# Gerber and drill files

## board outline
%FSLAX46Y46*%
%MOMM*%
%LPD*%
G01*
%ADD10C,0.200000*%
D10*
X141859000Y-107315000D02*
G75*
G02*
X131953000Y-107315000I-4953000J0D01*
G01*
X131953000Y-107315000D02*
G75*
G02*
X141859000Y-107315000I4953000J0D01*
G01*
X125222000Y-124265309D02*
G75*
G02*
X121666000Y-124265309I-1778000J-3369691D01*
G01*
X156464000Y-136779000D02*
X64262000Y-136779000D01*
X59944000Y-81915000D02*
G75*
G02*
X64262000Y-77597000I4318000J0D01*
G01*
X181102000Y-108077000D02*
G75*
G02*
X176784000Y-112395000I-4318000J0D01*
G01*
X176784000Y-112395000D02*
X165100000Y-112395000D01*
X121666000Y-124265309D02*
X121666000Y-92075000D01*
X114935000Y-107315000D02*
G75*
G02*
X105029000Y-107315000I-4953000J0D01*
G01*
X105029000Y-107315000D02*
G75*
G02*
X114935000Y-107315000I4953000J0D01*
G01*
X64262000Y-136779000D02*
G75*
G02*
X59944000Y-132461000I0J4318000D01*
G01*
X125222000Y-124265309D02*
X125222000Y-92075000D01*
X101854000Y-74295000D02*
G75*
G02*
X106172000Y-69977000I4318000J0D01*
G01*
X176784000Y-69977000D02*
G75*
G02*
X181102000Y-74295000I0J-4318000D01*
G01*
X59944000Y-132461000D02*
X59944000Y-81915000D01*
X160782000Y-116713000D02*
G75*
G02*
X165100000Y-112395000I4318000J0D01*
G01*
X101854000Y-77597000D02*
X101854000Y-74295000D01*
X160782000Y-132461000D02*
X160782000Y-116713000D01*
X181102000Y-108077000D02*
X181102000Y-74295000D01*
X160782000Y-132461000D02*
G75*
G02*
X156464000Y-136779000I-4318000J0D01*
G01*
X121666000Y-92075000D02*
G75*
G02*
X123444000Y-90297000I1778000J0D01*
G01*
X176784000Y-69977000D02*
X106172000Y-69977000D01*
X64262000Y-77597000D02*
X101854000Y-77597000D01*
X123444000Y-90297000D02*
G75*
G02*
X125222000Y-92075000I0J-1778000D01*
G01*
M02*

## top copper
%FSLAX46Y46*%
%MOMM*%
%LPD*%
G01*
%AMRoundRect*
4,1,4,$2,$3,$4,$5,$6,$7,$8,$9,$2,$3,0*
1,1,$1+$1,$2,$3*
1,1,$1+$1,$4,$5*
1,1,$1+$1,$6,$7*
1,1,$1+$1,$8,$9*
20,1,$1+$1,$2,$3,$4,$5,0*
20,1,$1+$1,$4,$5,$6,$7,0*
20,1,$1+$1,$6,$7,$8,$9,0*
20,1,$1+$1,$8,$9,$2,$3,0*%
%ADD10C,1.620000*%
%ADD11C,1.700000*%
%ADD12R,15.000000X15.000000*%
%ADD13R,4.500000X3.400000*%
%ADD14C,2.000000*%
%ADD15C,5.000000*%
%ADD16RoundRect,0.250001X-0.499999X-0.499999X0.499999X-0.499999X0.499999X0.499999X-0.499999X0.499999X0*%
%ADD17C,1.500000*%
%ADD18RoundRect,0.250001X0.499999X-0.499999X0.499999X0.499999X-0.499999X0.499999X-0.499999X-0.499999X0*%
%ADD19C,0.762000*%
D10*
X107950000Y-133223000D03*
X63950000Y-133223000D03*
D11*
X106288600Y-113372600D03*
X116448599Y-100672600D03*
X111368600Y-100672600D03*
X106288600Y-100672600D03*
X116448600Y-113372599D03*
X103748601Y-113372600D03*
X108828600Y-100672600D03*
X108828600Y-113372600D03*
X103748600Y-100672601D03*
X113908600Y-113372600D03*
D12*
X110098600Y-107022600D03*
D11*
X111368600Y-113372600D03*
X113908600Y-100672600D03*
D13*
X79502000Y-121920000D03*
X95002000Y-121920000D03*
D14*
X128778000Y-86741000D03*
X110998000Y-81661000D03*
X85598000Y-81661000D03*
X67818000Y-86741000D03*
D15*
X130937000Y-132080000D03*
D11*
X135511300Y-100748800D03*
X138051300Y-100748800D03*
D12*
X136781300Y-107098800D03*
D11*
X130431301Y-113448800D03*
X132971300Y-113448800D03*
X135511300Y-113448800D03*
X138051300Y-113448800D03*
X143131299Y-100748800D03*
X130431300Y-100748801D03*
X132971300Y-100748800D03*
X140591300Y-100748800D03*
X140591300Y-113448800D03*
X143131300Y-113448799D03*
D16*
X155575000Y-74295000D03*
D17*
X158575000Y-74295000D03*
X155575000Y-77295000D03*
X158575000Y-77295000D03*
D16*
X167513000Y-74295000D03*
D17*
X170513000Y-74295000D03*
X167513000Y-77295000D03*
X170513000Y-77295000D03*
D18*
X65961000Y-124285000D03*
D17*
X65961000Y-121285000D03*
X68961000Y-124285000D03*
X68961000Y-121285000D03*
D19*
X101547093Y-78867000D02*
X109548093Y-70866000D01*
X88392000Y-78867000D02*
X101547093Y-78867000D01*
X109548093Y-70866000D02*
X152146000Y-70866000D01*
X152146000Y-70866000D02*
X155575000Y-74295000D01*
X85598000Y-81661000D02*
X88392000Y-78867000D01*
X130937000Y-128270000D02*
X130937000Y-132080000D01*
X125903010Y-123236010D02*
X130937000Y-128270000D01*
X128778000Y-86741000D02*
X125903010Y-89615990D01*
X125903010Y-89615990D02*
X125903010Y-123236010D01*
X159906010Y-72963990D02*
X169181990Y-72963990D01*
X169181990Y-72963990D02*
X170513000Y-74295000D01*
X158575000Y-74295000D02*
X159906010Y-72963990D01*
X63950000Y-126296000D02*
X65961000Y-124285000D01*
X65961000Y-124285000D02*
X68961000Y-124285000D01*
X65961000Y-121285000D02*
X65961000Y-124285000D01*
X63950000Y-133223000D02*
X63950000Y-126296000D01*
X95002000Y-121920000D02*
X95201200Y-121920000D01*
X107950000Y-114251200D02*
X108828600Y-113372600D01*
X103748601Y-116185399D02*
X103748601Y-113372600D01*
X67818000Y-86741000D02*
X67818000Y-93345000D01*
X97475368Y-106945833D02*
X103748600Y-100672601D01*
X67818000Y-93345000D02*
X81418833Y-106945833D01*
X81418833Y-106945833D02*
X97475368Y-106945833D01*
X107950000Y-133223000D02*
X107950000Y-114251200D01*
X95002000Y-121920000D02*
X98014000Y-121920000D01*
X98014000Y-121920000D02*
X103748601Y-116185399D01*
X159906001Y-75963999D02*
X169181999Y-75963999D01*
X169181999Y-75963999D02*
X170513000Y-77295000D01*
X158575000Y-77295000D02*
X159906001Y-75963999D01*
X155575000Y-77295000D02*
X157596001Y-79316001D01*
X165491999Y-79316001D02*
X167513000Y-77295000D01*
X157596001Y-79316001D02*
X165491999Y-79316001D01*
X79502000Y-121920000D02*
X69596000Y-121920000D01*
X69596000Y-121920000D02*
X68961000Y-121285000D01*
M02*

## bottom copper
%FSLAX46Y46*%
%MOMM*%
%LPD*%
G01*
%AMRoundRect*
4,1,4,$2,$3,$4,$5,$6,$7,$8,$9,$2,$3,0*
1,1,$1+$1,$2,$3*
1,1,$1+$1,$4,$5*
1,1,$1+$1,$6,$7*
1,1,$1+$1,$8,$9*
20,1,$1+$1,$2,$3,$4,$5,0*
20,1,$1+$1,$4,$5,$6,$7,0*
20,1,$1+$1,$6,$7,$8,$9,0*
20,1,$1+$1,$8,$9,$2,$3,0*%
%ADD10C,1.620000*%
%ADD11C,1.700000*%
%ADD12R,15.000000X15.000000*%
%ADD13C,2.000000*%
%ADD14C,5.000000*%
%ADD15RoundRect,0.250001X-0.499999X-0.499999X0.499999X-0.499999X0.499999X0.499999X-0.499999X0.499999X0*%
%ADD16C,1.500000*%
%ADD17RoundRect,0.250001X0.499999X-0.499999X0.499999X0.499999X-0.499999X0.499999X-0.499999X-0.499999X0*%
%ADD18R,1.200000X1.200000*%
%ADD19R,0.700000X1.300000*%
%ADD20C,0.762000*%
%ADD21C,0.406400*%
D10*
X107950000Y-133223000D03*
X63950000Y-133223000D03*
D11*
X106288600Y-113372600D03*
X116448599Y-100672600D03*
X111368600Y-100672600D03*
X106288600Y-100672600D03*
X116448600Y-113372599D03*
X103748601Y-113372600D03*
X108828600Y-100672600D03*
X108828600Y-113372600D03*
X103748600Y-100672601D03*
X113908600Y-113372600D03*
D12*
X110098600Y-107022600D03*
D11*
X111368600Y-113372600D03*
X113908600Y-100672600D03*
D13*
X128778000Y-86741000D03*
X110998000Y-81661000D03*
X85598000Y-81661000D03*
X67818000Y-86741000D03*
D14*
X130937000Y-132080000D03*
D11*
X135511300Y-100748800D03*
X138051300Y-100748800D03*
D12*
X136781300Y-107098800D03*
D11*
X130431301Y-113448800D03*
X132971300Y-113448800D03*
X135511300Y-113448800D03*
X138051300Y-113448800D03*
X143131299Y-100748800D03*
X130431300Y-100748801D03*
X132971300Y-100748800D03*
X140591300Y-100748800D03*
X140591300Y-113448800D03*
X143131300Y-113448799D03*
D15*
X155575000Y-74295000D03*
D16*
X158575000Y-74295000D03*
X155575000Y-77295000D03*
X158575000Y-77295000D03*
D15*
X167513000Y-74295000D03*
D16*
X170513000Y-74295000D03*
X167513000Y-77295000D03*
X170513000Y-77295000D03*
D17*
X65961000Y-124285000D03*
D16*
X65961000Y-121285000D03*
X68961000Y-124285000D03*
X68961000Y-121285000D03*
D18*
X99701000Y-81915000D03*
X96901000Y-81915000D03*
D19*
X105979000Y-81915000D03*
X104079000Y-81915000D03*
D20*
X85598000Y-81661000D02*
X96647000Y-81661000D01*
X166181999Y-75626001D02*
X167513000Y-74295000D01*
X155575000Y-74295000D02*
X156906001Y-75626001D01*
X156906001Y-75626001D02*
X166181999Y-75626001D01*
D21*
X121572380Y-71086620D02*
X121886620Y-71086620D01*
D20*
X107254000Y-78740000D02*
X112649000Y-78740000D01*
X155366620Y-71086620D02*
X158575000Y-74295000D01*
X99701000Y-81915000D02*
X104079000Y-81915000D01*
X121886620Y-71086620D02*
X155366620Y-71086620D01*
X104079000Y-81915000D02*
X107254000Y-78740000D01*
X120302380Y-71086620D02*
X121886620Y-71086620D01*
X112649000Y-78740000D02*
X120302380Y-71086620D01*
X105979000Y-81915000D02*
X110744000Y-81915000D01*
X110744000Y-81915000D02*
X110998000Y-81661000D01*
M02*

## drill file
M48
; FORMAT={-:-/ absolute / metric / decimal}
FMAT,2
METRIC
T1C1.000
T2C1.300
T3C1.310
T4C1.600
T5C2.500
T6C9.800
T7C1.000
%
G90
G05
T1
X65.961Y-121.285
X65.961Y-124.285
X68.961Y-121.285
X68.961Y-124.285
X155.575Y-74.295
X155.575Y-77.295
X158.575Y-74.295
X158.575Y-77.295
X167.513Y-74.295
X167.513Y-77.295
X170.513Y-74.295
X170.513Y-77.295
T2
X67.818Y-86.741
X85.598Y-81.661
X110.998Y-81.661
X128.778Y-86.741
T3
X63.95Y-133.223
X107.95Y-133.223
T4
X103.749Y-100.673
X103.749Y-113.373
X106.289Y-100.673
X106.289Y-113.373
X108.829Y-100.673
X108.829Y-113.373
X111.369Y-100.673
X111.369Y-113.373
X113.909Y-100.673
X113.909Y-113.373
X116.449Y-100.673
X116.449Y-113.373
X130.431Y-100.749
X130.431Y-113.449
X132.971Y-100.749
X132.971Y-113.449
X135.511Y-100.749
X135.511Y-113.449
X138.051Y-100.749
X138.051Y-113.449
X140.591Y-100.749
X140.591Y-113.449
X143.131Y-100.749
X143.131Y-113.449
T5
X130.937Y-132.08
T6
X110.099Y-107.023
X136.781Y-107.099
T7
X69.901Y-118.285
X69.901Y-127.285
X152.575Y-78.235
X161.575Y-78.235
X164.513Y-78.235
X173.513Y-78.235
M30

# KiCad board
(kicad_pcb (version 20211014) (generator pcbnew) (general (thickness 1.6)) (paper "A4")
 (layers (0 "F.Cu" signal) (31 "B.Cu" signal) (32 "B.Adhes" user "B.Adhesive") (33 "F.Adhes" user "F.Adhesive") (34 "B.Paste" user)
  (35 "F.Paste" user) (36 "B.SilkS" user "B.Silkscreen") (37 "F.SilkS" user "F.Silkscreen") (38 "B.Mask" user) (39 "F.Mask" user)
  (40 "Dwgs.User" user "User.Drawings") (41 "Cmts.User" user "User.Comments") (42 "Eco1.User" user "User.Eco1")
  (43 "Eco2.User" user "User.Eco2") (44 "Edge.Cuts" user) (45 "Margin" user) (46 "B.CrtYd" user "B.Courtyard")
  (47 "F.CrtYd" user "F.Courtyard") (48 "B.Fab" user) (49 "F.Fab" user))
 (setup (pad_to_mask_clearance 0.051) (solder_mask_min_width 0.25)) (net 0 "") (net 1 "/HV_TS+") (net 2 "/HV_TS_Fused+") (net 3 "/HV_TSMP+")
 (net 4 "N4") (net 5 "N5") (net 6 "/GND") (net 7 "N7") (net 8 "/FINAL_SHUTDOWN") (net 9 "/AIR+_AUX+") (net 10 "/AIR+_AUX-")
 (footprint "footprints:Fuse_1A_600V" (layer "F.Cu") (at 107.95 133.223 180)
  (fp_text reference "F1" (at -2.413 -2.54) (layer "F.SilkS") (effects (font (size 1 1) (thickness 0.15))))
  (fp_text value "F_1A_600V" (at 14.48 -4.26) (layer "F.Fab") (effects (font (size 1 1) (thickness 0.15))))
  (pad "1" thru_hole circle locked (at 0 0 180) (size 1.62 1.62) (drill 1.31) (layers *.Cu *.Mask) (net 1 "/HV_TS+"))
  (pad "2" thru_hole circle locked (at 44 0 180) (size 1.62 1.62) (drill 1.31) (layers *.Cu *.Mask) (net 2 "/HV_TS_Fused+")))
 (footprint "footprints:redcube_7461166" (layer "F.Cu") (at 110.0986 107.0226)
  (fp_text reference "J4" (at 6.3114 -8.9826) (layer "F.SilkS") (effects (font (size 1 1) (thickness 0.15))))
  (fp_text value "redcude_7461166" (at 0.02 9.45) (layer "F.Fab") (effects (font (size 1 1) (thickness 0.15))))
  (pad "1" thru_hole circle locked (at -3.81 6.35) (size 1.7 1.7) (drill 1.6) (layers *.Cu *.Mask) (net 1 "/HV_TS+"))
  (pad "1" thru_hole circle locked (at 6.349999 -6.35) (size 1.7 1.7) (drill 1.6) (layers *.Cu *.Mask) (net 1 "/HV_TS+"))
  (pad "1" thru_hole circle locked (at 1.27 -6.35) (size 1.7 1.7) (drill 1.6) (layers *.Cu *.Mask) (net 1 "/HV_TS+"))
  (pad "1" thru_hole circle locked (at -3.81 -6.35) (size 1.7 1.7) (drill 1.6) (layers *.Cu *.Mask) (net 1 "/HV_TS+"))
  (pad "1" thru_hole circle locked (at 6.35 6.349999) (size 1.7 1.7) (drill 1.6) (layers *.Cu *.Mask) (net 1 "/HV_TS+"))
  (pad "1" thru_hole circle locked (at -6.349999 6.35) (size 1.7 1.7) (drill 1.6) (layers *.Cu *.Mask) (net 1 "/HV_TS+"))
  (pad "1" thru_hole circle locked (at -1.27 -6.35) (size 1.7 1.7) (drill 1.6) (layers *.Cu *.Mask) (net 1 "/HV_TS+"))
  (pad "1" thru_hole circle locked (at -1.27 6.35) (size 1.7 1.7) (drill 1.6) (layers *.Cu *.Mask) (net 1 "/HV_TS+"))
  (pad "1" thru_hole circle locked (at -6.35 -6.349999) (size 1.7 1.7) (drill 1.6) (layers *.Cu *.Mask) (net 1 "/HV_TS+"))
  (pad "1" thru_hole circle locked (at 3.81 6.35) (size 1.7 1.7) (drill 1.6) (layers *.Cu *.Mask) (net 1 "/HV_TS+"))
  (pad "1" thru_hole rect locked (at 0 0) (size 15 15) (drill 9.8) (layers *.Cu *.Mask) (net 1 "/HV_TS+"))
  (pad "1" thru_hole circle locked (at 1.27 6.35) (size 1.7 1.7) (drill 1.6) (layers *.Cu *.Mask) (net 1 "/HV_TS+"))
  (pad "1" thru_hole circle locked (at 3.81 -6.35) (size 1.7 1.7) (drill 1.6) (layers *.Cu *.Mask) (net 1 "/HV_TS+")))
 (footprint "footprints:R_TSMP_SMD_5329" (layer "F.Cu") (at 87.122 121.92)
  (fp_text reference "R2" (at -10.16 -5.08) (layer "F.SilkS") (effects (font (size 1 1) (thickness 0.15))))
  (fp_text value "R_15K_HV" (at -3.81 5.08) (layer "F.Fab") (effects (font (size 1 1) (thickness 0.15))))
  (pad "1" smd rect locked (at -7.62 0) (size 4.5 3.4) (layers "F.Cu" "F.Paste" "F.Mask") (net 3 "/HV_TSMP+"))
  (pad "2" smd rect locked (at 7.88 0) (size 4.5 3.4) (layers "F.Cu" "F.Paste" "F.Mask") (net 1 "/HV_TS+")))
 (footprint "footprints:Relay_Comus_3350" (layer "F.Cu") (at 64.008 94.234)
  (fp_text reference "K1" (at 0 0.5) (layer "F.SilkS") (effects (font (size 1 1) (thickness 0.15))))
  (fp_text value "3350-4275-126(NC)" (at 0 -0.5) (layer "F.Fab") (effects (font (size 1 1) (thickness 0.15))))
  (pad "1" thru_hole circle locked (at 64.77 -7.493) (size 2 2) (drill 1.3) (layers *.Cu *.Mask) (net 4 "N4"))
  (pad "2" thru_hole circle locked (at 46.99 -12.573) (size 2 2) (drill 1.3) (layers *.Cu *.Mask) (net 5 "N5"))
  (pad "3" thru_hole circle locked (at 21.59 -12.573) (size 2 2) (drill 1.3) (layers *.Cu *.Mask) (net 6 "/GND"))
  (pad "4" thru_hole circle locked (at 3.81 -7.493) (size 2 2) (drill 1.3) (layers *.Cu *.Mask) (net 1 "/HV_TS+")))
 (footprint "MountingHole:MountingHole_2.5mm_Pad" (layer "F.Cu") (at 130.937 132.08 -90)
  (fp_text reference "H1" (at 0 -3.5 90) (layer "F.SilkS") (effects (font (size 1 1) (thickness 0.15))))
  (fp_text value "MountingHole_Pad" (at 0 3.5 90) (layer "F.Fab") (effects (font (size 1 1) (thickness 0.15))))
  (pad "1" thru_hole circle (at 0 0 270) (size 5 5) (drill 2.5) (layers *.Cu *.Mask) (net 4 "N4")))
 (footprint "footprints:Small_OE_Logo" (layer "F.Cu") (at 153.416 107.188)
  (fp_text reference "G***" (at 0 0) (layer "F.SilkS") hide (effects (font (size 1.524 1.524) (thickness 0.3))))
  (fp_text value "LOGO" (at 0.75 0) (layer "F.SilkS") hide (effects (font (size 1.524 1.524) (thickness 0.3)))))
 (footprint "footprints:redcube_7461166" (layer "F.Cu") (at 136.7813 107.0988)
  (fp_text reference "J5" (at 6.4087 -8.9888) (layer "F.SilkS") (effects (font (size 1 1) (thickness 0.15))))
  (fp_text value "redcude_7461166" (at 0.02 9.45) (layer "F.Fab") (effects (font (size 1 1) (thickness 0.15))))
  (pad "1" thru_hole circle locked (at -1.27 -6.35) (size 1.7 1.7) (drill 1.6) (layers *.Cu *.Mask) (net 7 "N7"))
  (pad "1" thru_hole circle locked (at 1.27 -6.35) (size 1.7 1.7) (drill 1.6) (layers *.Cu *.Mask) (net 7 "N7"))
  (pad "1" thru_hole rect locked (at 0 0) (size 15 15) (drill 9.8) (layers *.Cu *.Mask) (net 7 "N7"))
  (pad "1" thru_hole circle locked (at -6.349999 6.35) (size 1.7 1.7) (drill 1.6) (layers *.Cu *.Mask) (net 7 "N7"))
  (pad "1" thru_hole circle locked (at -3.81 6.35) (size 1.7 1.7) (drill 1.6) (layers *.Cu *.Mask) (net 7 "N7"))
  (pad "1" thru_hole circle locked (at -1.27 6.35) (size 1.7 1.7) (drill 1.6) (layers *.Cu *.Mask) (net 7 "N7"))
  (pad "1" thru_hole circle locked (at 1.27 6.35) (size 1.7 1.7) (drill 1.6) (layers *.Cu *.Mask) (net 7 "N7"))
  (pad "1" thru_hole circle locked (at 6.349999 -6.35) (size 1.7 1.7) (drill 1.6) (layers *.Cu *.Mask) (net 7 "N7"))
  (pad "1" thru_hole circle locked (at -6.35 -6.349999) (size 1.7 1.7) (drill 1.6) (layers *.Cu *.Mask) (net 7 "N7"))
  (pad "1" thru_hole circle locked (at -3.81 -6.35) (size 1.7 1.7) (drill 1.6) (layers *.Cu *.Mask) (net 7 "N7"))
  (pad "1" thru_hole circle locked (at 3.81 -6.35) (size 1.7 1.7) (drill 1.6) (layers *.Cu *.Mask) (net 7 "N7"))
  (pad "1" thru_hole circle locked (at 3.81 6.35) (size 1.7 1.7) (drill 1.6) (layers *.Cu *.Mask) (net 7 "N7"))
  (pad "1" thru_hole circle locked (at 6.35 6.349999) (size 1.7 1.7) (drill 1.6) (layers *.Cu *.Mask) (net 7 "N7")))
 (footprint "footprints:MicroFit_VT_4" (layer "F.Cu") (at 155.575 74.295)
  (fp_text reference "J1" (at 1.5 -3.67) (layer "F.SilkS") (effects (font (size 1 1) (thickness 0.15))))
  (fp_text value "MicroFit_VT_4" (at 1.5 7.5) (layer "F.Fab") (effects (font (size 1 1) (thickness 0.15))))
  (pad "" np_thru_hole circle locked (at 6 3.94) (size 1 1) (drill 1) (layers *.Cu *.Mask))
  (pad "" np_thru_hole circle locked (at -3 3.94) (size 1 1) (drill 1) (layers *.Cu *.Mask))
  (pad "1" thru_hole roundrect locked (at 0 0) (size 1.5 1.5) (drill 1) (layers *.Cu *.Mask) (roundrect_rratio 0.166667) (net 6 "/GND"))
  (pad "2" thru_hole circle locked (at 3 0) (size 1.5 1.5) (drill 1) (layers *.Cu *.Mask) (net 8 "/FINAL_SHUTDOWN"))
  (pad "3" thru_hole circle locked (at 0 3) (size 1.5 1.5) (drill 1) (layers *.Cu *.Mask) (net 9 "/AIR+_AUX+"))
  (pad "4" thru_hole circle locked (at 3 3) (size 1.5 1.5) (drill 1) (layers *.Cu *.Mask) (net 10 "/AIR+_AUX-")))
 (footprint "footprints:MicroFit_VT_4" (layer "F.Cu") (at 167.513 74.295)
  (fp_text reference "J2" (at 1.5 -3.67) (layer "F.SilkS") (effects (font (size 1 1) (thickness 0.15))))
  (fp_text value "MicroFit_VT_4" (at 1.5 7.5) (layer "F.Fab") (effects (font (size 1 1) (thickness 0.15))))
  (pad "" np_thru_hole circle locked (at 6 3.94) (size 1 1) (drill 1) (layers *.Cu *.Mask))
  (pad "" np_thru_hole circle locked (at -3 3.94) (size 1 1) (drill 1) (layers *.Cu *.Mask))
  (pad "1" thru_hole roundrect locked (at 0 0) (size 1.5 1.5) (drill 1) (layers *.Cu *.Mask) (roundrect_rratio 0.166667) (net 6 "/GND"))
  (pad "2" thru_hole circle locked (at 3 0) (size 1.5 1.5) (drill 1) (layers *.Cu *.Mask) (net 8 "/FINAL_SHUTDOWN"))
  (pad "3" thru_hole circle locked (at 0 3) (size 1.5 1.5) (drill 1) (layers *.Cu *.Mask) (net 9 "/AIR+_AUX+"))
  (pad "4" thru_hole circle locked (at 3 3) (size 1.5 1.5) (drill 1) (layers *.Cu *.Mask) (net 10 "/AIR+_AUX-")))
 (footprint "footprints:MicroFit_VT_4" (layer "F.Cu") (at 65.961 124.285 90)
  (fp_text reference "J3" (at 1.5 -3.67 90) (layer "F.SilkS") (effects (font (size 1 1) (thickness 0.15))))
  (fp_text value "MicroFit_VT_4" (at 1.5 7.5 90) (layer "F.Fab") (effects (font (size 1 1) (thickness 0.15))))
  (pad "" np_thru_hole circle locked (at -3 3.94 90) (size 1 1) (drill 1) (layers *.Cu *.Mask))
  (pad "" np_thru_hole circle locked (at 6 3.94 90) (size 1 1) (drill 1) (layers *.Cu *.Mask))
  (pad "1" thru_hole roundrect locked (at 0 0 90) (size 1.5 1.5) (drill 1) (layers *.Cu *.Mask) (roundrect_rratio 0.166667)
   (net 2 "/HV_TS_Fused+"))
  (pad "2" thru_hole circle locked (at 3 0 90) (size 1.5 1.5) (drill 1) (layers *.Cu *.Mask) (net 2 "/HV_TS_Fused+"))
  (pad "3" thru_hole circle locked (at 0 3 90) (size 1.5 1.5) (drill 1) (layers *.Cu *.Mask) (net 2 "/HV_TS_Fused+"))
  (pad "4" thru_hole circle locked (at 3 3 90) (size 1.5 1.5) (drill 1) (layers *.Cu *.Mask) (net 3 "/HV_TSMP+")))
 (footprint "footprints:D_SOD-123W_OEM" (layer "B.Cu") (at 98.301 81.915 180)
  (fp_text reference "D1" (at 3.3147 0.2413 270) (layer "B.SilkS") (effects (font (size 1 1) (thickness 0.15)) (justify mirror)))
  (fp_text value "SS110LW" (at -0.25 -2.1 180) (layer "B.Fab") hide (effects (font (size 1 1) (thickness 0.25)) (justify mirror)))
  (pad "1" smd rect locked (at -1.4 0 180) (size 1.2 1.2) (layers "B.Cu" "B.Paste" "B.Mask") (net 8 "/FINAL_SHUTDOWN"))
  (pad "2" smd rect locked (at 1.4 0 180) (size 1.2 1.2) (layers "B.Cu" "B.Paste" "B.Mask") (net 6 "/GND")))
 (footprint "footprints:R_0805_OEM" (layer "B.Cu") (at 105.029 81.915 180)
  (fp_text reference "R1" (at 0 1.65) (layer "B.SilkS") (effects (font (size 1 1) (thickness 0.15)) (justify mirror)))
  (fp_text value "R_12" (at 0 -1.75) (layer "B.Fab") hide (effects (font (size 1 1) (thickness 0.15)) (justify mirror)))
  (pad "1" smd rect locked (at -0.95 0 180) (size 0.7 1.3) (layers "B.Cu" "B.Paste" "B.Mask") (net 5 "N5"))
  (pad "2" smd rect locked (at 0.95 0 180) (size 0.7 1.3) (layers "B.Cu" "B.Paste" "B.Mask") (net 8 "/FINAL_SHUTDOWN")))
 (gr_circle (center 136.906 107.315) (end 131.953 107.315) (layer "Edge.Cuts") (width 0.2) (fill none))
 (gr_arc (start 125.222 124.265309) (mid 123.444 131.445) (end 121.666 124.265309) (layer "Edge.Cuts") (width 0.2))
 (gr_line (start 156.464 136.779) (end 64.262 136.779) (layer "Edge.Cuts") (width 0.2))
 (gr_arc (start 59.944 81.915) (mid 61.208713 78.861713) (end 64.262 77.597) (layer "Edge.Cuts") (width 0.2))
 (gr_arc (start 181.102 108.077) (mid 179.837287 111.130287) (end 176.784 112.395) (layer "Edge.Cuts") (width 0.2))
 (gr_line (start 176.784 112.395) (end 165.1 112.395) (layer "Edge.Cuts") (width 0.2))
 (gr_line (start 121.666 124.265309) (end 121.666 92.075) (layer "Edge.Cuts") (width 0.2))
 (gr_circle (center 109.982 107.315) (end 105.029 107.315) (layer "Edge.Cuts") (width 0.2) (fill none))
 (gr_arc (start 64.262 136.779) (mid 61.208713 135.514287) (end 59.944 132.461) (layer "Edge.Cuts") (width 0.2))
 (gr_line (start 125.222 124.265309) (end 125.222 92.075) (layer "Edge.Cuts") (width 0.2))
 (gr_arc (start 101.854 74.295) (mid 103.118713 71.241713) (end 106.172 69.977) (layer "Edge.Cuts") (width 0.2))
 (gr_arc (start 176.784 69.977) (mid 179.837287 71.241713) (end 181.102 74.295) (layer "Edge.Cuts") (width 0.2))
 (gr_line (start 59.944 132.461) (end 59.944 81.915) (layer "Edge.Cuts") (width 0.2))
 (gr_arc (start 160.782 116.713) (mid 162.046713 113.659713) (end 165.1 112.395) (layer "Edge.Cuts") (width 0.2))
 (gr_line (start 101.854 77.597) (end 101.854 74.295) (layer "Edge.Cuts") (width 0.2))
 (gr_line (start 160.782 132.461) (end 160.782 116.713) (layer "Edge.Cuts") (width 0.2))
 (gr_line (start 181.102 108.077) (end 181.102 74.295) (layer "Edge.Cuts") (width 0.2))
 (gr_arc (start 160.782 132.461) (mid 159.517287 135.514287) (end 156.464 136.779) (layer "Edge.Cuts") (width 0.2))
 (gr_arc (start 121.666 92.075) (mid 122.186764 90.817764) (end 123.444 90.297) (layer "Edge.Cuts") (width 0.2))
 (gr_line (start 176.784 69.977) (end 106.172 69.977) (layer "Edge.Cuts") (width 0.2))
 (gr_line (start 64.262 77.597) (end 101.854 77.597) (layer "Edge.Cuts") (width 0.2))
 (gr_arc (start 123.444 90.297) (mid 124.701236 90.817764) (end 125.222 92.075) (layer "Edge.Cuts") (width 0.2))
 (segment (start 101.547093 78.867) (end 109.548093 70.866) (width 0.762) (layer "F.Cu") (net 6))
 (segment (start 88.392 78.867) (end 101.547093 78.867) (width 0.762) (layer "F.Cu") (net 6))
 (segment (start 109.548093 70.866) (end 152.146 70.866) (width 0.762) (layer "F.Cu") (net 6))
 (segment (start 152.146 70.866) (end 155.575 74.295) (width 0.762) (layer "F.Cu") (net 6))
 (segment (start 85.598 81.661) (end 88.392 78.867) (width 0.762) (layer "F.Cu") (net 6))
 (segment (start 85.598 81.661) (end 96.647 81.661) (width 0.762) (layer "B.Cu") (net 6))
 (segment (start 166.181999 75.626001) (end 167.513 74.295) (width 0.762) (layer "B.Cu") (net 6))
 (segment (start 155.575 74.295) (end 156.906001 75.626001) (width 0.762) (layer "B.Cu") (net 6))
 (segment (start 156.906001 75.626001) (end 166.181999 75.626001) (width 0.762) (layer "B.Cu") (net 6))
 (segment (start 130.937 128.27) (end 130.937 132.08) (width 0.762) (layer "F.Cu") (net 4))
 (segment (start 125.90301 123.23601) (end 130.937 128.27) (width 0.762) (layer "F.Cu") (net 4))
 (segment (start 128.778 86.741) (end 125.90301 89.61599) (width 0.762) (layer "F.Cu") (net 4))
 (segment (start 125.90301 89.61599) (end 125.90301 123.23601) (width 0.762) (layer "F.Cu") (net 4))
 (segment (start 159.90601 72.96399) (end 169.18199 72.96399) (width 0.762) (layer "F.Cu") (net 8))
 (segment (start 169.18199 72.96399) (end 170.513 74.295) (width 0.762) (layer "F.Cu") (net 8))
 (segment (start 158.575 74.295) (end 159.90601 72.96399) (width 0.762) (layer "F.Cu") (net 8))
 (segment (start 121.57238 71.08662) (end 121.88662 71.08662) (width 0.4064) (layer "B.Cu") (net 8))
 (segment (start 107.254 78.74) (end 112.649 78.74) (width 0.762) (layer "B.Cu") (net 8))
 (segment (start 155.36662 71.08662) (end 158.575 74.295) (width 0.762) (layer "B.Cu") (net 8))
 (segment (start 99.701 81.915) (end 104.079 81.915) (width 0.762) (layer "B.Cu") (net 8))
 (segment (start 121.88662 71.08662) (end 155.36662 71.08662) (width 0.762) (layer "B.Cu") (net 8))
 (segment (start 104.079 81.915) (end 107.254 78.74) (width 0.762) (layer "B.Cu") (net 8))
 (segment (start 120.30238 71.08662) (end 121.88662 71.08662) (width 0.762) (layer "B.Cu") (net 8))
 (segment (start 112.649 78.74) (end 120.30238 71.08662) (width 0.762) (layer "B.Cu") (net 8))
 (segment (start 63.95 126.296) (end 65.961 124.285) (width 0.762) (layer "F.Cu") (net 2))
 (segment (start 65.961 124.285) (end 68.961 124.285) (width 0.762) (layer "F.Cu") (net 2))
 (segment (start 65.961 121.285) (end 65.961 124.285) (width 0.762) (layer "F.Cu") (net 2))
 (segment (start 63.95 133.223) (end 63.95 126.296) (width 0.762) (layer "F.Cu") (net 2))
 (segment (start 95.002 121.92) (end 95.2012 121.92) (width 0.762) (layer "F.Cu") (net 1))
 (segment (start 107.95 114.2512) (end 108.8286 113.3726) (width 0.762) (layer "F.Cu") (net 1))
 (segment (start 103.748601 116.185399) (end 103.748601 113.3726) (width 0.762) (layer "F.Cu") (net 1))
 (segment (start 67.818 86.741) (end 67.818 93.345) (width 0.762) (layer "F.Cu") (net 1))
 (segment (start 97.475368 106.945833) (end 103.7486 100.672601) (width 0.762) (layer "F.Cu") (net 1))
 (segment (start 67.818 93.345) (end 81.418833 106.945833) (width 0.762) (layer "F.Cu") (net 1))
 (segment (start 81.418833 106.945833) (end 97.475368 106.945833) (width 0.762) (layer "F.Cu") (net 1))
 (segment (start 107.95 133.223) (end 107.95 114.2512) (width 0.762) (layer "F.Cu") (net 1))
 (segment (start 95.002 121.92) (end 98.014 121.92) (width 0.762) (layer "F.Cu") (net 1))
 (segment (start 98.014 121.92) (end 103.748601 116.185399) (width 0.762) (layer "F.Cu") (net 1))
 (segment (start 159.906001 75.963999) (end 169.181999 75.963999) (width 0.762) (layer "F.Cu") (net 10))
 (segment (start 169.181999 75.963999) (end 170.513 77.295) (width 0.762) (layer "F.Cu") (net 10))
 (segment (start 158.575 77.295) (end 159.906001 75.963999) (width 0.762) (layer "F.Cu") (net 10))
 (segment (start 155.575 77.295) (end 157.596001 79.316001) (width 0.762) (layer "F.Cu") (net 9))
 (segment (start 165.491999 79.316001) (end 167.513 77.295) (width 0.762) (layer "F.Cu") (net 9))
 (segment (start 157.596001 79.316001) (end 165.491999 79.316001) (width 0.762) (layer "F.Cu") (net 9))
 (segment (start 79.502 121.92) (end 69.596 121.92) (width 0.762) (layer "F.Cu") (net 3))
 (segment (start 69.596 121.92) (end 68.961 121.285) (width 0.762) (layer "F.Cu") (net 3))
 (segment (start 105.979 81.915) (end 110.744 81.915) (width 0.762) (layer "B.Cu") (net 5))
 (segment (start 110.744 81.915) (end 110.998 81.661) (width 0.762) (layer "B.Cu") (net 5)))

